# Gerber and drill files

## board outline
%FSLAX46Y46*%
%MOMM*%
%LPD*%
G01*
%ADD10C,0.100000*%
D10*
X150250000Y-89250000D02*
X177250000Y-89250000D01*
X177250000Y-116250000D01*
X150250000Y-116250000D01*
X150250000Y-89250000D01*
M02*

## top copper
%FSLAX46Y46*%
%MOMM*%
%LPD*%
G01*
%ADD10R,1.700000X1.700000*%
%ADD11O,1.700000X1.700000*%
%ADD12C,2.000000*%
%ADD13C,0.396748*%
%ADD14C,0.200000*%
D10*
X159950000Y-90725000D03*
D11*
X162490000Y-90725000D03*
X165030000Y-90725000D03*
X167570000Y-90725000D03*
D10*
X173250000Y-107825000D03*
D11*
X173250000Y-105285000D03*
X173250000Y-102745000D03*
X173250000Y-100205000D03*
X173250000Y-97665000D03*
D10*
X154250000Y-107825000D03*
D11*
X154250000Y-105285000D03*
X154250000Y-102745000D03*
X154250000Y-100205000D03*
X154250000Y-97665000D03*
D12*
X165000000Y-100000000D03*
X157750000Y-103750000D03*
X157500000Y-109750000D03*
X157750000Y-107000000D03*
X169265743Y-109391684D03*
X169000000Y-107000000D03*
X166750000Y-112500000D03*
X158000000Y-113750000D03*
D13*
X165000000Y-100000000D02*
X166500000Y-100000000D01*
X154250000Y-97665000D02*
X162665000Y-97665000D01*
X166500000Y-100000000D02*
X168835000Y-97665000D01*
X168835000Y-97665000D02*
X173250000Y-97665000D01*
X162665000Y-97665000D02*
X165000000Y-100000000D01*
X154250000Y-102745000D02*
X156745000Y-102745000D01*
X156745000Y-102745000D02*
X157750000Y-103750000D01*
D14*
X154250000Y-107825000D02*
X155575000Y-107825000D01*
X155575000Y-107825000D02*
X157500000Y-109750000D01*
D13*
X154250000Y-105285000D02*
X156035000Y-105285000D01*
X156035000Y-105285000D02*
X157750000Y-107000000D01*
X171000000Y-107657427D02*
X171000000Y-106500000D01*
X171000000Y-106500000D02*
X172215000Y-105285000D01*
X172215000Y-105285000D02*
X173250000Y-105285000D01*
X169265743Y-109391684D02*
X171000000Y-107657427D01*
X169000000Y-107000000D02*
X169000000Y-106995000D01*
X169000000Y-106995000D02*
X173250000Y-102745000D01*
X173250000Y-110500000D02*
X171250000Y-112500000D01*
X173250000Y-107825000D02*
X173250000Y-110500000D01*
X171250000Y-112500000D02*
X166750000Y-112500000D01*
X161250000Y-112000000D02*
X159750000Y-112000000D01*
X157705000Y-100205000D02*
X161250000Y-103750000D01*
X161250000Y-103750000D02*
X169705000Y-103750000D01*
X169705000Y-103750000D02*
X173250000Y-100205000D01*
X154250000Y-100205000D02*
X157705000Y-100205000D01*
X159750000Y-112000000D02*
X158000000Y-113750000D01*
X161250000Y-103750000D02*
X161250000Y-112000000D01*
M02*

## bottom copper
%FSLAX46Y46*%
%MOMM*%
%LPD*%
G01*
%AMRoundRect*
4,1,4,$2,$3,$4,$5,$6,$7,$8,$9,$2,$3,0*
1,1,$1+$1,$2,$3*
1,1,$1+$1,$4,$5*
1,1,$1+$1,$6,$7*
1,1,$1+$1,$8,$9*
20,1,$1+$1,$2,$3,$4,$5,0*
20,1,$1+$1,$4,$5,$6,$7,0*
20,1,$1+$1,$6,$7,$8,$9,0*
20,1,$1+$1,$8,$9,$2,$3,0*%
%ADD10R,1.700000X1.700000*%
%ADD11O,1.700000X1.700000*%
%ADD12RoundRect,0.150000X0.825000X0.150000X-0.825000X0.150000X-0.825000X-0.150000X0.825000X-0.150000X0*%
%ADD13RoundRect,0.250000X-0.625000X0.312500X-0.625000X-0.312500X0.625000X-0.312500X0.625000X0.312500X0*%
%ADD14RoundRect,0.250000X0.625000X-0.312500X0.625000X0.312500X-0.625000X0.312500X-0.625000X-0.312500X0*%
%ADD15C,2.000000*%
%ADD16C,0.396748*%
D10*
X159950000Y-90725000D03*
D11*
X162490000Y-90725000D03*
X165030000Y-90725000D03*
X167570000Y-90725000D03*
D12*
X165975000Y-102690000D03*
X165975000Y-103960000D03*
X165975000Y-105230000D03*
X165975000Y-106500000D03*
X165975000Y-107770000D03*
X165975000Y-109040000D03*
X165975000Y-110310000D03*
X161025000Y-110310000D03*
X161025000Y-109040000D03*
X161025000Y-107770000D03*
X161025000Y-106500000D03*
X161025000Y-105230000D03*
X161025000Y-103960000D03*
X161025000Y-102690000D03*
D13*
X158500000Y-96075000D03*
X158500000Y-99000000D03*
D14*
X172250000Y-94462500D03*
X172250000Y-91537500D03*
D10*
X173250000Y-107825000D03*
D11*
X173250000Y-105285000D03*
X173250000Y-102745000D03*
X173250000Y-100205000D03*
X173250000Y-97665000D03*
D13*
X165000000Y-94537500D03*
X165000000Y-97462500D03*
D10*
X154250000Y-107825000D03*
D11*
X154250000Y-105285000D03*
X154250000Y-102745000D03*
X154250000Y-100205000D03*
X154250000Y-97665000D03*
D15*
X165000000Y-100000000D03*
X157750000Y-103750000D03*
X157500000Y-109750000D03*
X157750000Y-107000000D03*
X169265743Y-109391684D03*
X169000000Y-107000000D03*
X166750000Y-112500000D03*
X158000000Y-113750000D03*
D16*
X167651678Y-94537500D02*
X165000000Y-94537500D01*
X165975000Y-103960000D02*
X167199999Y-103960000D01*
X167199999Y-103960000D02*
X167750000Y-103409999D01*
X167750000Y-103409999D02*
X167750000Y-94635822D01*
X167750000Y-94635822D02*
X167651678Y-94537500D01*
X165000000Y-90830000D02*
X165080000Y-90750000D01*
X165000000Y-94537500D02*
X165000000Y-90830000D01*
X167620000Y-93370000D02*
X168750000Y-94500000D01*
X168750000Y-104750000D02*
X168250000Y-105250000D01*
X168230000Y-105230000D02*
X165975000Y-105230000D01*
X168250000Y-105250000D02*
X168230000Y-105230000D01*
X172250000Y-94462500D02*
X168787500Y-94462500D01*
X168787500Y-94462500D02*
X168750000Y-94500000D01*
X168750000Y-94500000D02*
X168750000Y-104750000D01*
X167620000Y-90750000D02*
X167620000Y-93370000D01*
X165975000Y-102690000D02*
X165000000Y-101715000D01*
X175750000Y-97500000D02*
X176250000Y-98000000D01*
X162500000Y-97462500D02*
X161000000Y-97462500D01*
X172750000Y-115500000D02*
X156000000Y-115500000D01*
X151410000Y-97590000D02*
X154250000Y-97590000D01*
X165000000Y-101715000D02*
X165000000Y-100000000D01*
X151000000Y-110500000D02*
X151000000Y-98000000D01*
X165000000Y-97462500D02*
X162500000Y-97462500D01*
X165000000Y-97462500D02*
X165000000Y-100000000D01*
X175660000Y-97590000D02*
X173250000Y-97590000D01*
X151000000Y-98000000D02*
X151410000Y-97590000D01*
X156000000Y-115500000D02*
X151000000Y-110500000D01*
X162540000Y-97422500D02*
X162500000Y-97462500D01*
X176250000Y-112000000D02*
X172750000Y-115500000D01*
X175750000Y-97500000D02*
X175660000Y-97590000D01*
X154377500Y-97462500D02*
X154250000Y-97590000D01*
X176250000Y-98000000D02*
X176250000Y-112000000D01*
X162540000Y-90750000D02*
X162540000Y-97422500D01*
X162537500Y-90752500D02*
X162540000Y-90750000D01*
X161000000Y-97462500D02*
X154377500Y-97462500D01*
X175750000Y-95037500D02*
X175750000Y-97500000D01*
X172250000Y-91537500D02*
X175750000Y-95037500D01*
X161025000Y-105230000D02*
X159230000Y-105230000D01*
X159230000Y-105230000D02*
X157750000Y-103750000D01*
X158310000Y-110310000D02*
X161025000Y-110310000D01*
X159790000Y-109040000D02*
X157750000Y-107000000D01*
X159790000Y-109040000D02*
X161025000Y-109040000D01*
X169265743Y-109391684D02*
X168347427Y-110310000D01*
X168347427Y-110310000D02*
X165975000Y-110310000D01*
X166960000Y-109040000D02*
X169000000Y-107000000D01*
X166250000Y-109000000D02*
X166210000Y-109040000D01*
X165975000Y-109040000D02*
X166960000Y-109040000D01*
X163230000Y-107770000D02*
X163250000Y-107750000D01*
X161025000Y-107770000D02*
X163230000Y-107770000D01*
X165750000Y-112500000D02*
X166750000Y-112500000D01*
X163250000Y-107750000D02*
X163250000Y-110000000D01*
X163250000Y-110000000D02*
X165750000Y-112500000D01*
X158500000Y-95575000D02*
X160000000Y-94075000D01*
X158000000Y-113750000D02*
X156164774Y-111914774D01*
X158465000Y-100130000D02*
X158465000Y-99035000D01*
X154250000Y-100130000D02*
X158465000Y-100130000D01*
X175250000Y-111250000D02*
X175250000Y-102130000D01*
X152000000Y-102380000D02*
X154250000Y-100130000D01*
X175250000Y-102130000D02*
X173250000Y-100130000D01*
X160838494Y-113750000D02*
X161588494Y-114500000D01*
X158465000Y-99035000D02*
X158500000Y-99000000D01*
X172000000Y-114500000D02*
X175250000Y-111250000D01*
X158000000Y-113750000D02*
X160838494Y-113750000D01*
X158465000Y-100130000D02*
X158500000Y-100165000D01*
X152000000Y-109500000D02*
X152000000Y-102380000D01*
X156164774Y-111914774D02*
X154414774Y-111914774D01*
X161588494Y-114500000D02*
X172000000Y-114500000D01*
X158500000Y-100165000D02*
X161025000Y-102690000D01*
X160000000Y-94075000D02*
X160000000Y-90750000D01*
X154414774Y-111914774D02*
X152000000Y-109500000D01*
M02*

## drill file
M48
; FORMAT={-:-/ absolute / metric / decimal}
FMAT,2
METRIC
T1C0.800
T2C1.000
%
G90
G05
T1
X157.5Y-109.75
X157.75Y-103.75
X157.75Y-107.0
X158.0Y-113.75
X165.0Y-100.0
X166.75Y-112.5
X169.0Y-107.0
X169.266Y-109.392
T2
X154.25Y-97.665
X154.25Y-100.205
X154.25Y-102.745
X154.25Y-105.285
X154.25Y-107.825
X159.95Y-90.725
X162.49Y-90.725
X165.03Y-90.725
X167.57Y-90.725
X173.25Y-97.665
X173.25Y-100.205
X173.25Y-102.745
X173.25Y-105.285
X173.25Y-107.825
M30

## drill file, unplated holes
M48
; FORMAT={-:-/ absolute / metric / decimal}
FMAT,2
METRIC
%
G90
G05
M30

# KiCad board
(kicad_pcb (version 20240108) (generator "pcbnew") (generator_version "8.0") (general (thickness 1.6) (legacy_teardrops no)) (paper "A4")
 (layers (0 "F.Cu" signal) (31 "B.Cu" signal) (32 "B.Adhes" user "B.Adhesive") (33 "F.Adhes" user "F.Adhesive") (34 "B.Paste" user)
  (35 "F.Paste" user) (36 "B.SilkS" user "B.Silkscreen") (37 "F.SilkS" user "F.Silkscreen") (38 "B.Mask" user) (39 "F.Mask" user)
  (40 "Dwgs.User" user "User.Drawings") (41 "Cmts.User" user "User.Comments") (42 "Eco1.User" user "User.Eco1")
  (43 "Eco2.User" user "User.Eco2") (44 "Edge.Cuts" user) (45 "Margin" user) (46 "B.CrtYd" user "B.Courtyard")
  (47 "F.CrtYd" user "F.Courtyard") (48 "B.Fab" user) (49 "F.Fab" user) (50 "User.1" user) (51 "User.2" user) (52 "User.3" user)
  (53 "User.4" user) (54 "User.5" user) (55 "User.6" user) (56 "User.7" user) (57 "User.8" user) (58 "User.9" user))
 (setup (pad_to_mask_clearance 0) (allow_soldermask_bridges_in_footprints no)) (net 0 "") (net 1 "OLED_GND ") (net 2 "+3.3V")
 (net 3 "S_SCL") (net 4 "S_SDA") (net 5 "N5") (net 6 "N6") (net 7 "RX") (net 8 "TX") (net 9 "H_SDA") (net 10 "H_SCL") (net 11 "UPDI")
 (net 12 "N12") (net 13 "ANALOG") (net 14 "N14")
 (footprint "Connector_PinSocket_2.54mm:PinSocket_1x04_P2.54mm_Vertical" (layer "F.Cu") (at 159.95 90.725 90)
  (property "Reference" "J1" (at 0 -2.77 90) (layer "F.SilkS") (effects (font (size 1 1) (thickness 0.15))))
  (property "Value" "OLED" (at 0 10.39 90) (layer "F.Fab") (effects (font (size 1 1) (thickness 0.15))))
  (pad "1" thru_hole rect (at 0 0 90) (size 1.7 1.7) (drill 1) (layers "*.Cu" "*.Mask") (remove_unused_layers no) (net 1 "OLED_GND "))
  (pad "2" thru_hole oval (at 0 2.54 90) (size 1.7 1.7) (drill 1) (layers "*.Cu" "*.Mask") (remove_unused_layers no) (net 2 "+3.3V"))
  (pad "3" thru_hole oval (at 0 5.08 90) (size 1.7 1.7) (drill 1) (layers "*.Cu" "*.Mask") (remove_unused_layers no) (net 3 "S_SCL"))
  (pad "4" thru_hole oval (at 0 7.62 90) (size 1.7 1.7) (drill 1) (layers "*.Cu" "*.Mask") (remove_unused_layers no) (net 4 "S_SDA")))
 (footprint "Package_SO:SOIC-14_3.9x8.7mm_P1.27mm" (layer "B.Cu") (at 163.5 106.5 180)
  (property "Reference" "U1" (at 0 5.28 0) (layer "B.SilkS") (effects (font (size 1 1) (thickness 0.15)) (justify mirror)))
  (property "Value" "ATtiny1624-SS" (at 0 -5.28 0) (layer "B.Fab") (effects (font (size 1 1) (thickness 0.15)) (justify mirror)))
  (pad "1" smd roundrect (at -2.475 3.81 180) (size 1.95 0.6) (layers "B.Cu" "B.Paste" "B.Mask") (roundrect_rratio 0.25) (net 2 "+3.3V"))
  (pad "2" smd roundrect (at -2.475 2.54 180) (size 1.95 0.6) (layers "B.Cu" "B.Paste" "B.Mask") (roundrect_rratio 0.25) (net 3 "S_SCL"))
  (pad "3" smd roundrect (at -2.475 1.27 180) (size 1.95 0.6) (layers "B.Cu" "B.Paste" "B.Mask") (roundrect_rratio 0.25) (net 4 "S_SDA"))
  (pad "4" smd roundrect (at -2.475 0 180) (size 1.95 0.6) (layers "B.Cu" "B.Paste" "B.Mask") (roundrect_rratio 0.25) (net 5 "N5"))
  (pad "5" smd roundrect (at -2.475 -1.27 180) (size 1.95 0.6) (layers "B.Cu" "B.Paste" "B.Mask") (roundrect_rratio 0.25) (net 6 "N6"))
  (pad "6" smd roundrect (at -2.475 -2.54 180) (size 1.95 0.6) (layers "B.Cu" "B.Paste" "B.Mask") (roundrect_rratio 0.25) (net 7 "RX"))
  (pad "7" smd roundrect (at -2.475 -3.81 180) (size 1.95 0.6) (layers "B.Cu" "B.Paste" "B.Mask") (roundrect_rratio 0.25) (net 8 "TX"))
  (pad "8" smd roundrect (at 2.475 -3.81 180) (size 1.95 0.6) (layers "B.Cu" "B.Paste" "B.Mask") (roundrect_rratio 0.25) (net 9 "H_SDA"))
  (pad "9" smd roundrect (at 2.475 -2.54 180) (size 1.95 0.6) (layers "B.Cu" "B.Paste" "B.Mask") (roundrect_rratio 0.25) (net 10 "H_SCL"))
  (pad "10" smd roundrect (at 2.475 -1.27 180) (size 1.95 0.6) (layers "B.Cu" "B.Paste" "B.Mask") (roundrect_rratio 0.25) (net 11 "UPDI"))
  (pad "11" smd roundrect (at 2.475 0 180) (size 1.95 0.6) (layers "B.Cu" "B.Paste" "B.Mask") (roundrect_rratio 0.25) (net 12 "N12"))
  (pad "12" smd roundrect (at 2.475 1.27 180) (size 1.95 0.6) (layers "B.Cu" "B.Paste" "B.Mask") (roundrect_rratio 0.25) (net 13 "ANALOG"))
  (pad "13" smd roundrect (at 2.475 2.54 180) (size 1.95 0.6) (layers "B.Cu" "B.Paste" "B.Mask") (roundrect_rratio 0.25) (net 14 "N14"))
  (pad "14" smd roundrect (at 2.475 3.81 180) (size 1.95 0.6) (layers "B.Cu" "B.Paste" "B.Mask") (roundrect_rratio 0.25) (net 1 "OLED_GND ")))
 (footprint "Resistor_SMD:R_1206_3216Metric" (layer "B.Cu") (at 158.5 97.5375 -90)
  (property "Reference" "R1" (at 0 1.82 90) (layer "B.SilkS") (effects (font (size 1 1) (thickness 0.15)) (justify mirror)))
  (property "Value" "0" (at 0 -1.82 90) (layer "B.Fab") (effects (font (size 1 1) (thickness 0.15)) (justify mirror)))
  (pad "1" smd roundrect (at -1.4625 0 270) (size 1.125 1.75) (layers "B.Cu" "B.Paste" "B.Mask") (roundrect_rratio 0.222222)
   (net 1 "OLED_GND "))
  (pad "2" smd roundrect (at 1.4625 0 270) (size 1.125 1.75) (layers "B.Cu" "B.Paste" "B.Mask") (roundrect_rratio 0.222222)
   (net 1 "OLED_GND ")))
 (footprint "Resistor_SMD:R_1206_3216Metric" (layer "B.Cu") (at 172.25 93 90)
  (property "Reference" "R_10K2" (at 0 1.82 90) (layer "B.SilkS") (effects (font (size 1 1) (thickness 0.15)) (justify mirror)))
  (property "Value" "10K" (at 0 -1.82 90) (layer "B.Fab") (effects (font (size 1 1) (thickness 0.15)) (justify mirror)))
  (pad "1" smd roundrect (at -1.4625 0 90) (size 1.125 1.75) (layers "B.Cu" "B.Paste" "B.Mask") (roundrect_rratio 0.222222) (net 4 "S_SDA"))
  (pad "2" smd roundrect (at 1.4625 0 90) (size 1.125 1.75) (layers "B.Cu" "B.Paste" "B.Mask") (roundrect_rratio 0.222222) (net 2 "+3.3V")))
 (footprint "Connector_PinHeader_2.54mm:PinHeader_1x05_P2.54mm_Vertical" (layer "B.Cu") (at 173.25 107.825)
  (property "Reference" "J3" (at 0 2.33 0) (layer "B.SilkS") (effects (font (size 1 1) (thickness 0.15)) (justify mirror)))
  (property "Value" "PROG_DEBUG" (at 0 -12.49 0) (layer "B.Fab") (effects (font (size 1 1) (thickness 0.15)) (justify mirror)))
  (pad "1" thru_hole rect (at 0 0) (size 1.7 1.7) (drill 1) (layers "*.Cu" "*.Mask") (remove_unused_layers no) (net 11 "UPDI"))
  (pad "2" thru_hole oval (at 0 -2.54) (size 1.7 1.7) (drill 1) (layers "*.Cu" "*.Mask") (remove_unused_layers no) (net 8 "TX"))
  (pad "3" thru_hole oval (at 0 -5.08) (size 1.7 1.7) (drill 1) (layers "*.Cu" "*.Mask") (remove_unused_layers no) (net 7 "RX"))
  (pad "4" thru_hole oval (at 0 -7.62) (size 1.7 1.7) (drill 1) (layers "*.Cu" "*.Mask") (remove_unused_layers no) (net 1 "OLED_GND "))
  (pad "5" thru_hole oval (at 0 -10.16) (size 1.7 1.7) (drill 1) (layers "*.Cu" "*.Mask") (remove_unused_layers no) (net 2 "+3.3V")))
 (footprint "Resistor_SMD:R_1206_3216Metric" (layer "B.Cu") (at 165 96 -90)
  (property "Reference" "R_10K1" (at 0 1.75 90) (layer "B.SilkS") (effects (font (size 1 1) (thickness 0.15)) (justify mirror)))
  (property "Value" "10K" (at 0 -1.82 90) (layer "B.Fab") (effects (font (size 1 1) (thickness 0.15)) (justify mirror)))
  (pad "1" smd roundrect (at -1.4625 0 270) (size 1.125 1.75) (layers "B.Cu" "B.Paste" "B.Mask") (roundrect_rratio 0.222222) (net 3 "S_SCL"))
  (pad "2" smd roundrect (at 1.4625 0 270) (size 1.125 1.75) (layers "B.Cu" "B.Paste" "B.Mask") (roundrect_rratio 0.222222) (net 2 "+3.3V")))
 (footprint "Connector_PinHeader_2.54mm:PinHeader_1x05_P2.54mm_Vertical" (layer "B.Cu") (at 154.25 107.825)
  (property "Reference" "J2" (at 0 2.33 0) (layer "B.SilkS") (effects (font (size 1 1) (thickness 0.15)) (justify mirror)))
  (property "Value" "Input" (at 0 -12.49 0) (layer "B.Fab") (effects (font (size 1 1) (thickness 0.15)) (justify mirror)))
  (pad "1" thru_hole rect (at 0 0) (size 1.7 1.7) (drill 1) (layers "*.Cu" "*.Mask") (remove_unused_layers no) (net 9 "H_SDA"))
  (pad "2" thru_hole oval (at 0 -2.54) (size 1.7 1.7) (drill 1) (layers "*.Cu" "*.Mask") (remove_unused_layers no) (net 10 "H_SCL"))
  (pad "3" thru_hole oval (at 0 -5.08) (size 1.7 1.7) (drill 1) (layers "*.Cu" "*.Mask") (remove_unused_layers no) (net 13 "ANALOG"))
  (pad "4" thru_hole oval (at 0 -7.62) (size 1.7 1.7) (drill 1) (layers "*.Cu" "*.Mask") (remove_unused_layers no) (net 1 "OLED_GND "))
  (pad "5" thru_hole oval (at 0 -10.16) (size 1.7 1.7) (drill 1) (layers "*.Cu" "*.Mask") (remove_unused_layers no) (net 2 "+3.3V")))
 (gr_rect (start 150.25 89.25) (end 177.25 116.25) (stroke (width 0.1) (type default)) (fill none) (layer "Edge.Cuts"))
 (segment (start 167.651678 94.5375) (end 165 94.5375) (width 0.396748) (layer "B.Cu") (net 3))
 (segment (start 165.975 103.96) (end 167.199999 103.96) (width 0.396748) (layer "B.Cu") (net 3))
 (segment (start 167.199999 103.96) (end 167.75 103.409999) (width 0.396748) (layer "B.Cu") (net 3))
 (segment (start 167.75 103.409999) (end 167.75 94.635822) (width 0.396748) (layer "B.Cu") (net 3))
 (segment (start 167.75 94.635822) (end 167.651678 94.5375) (width 0.396748) (layer "B.Cu") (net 3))
 (segment (start 165 90.83) (end 165.08 90.75) (width 0.396748) (layer "B.Cu") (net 3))
 (segment (start 165 94.5375) (end 165 90.83) (width 0.396748) (layer "B.Cu") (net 3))
 (segment (start 167.62 93.37) (end 168.75 94.5) (width 0.396748) (layer "B.Cu") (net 4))
 (segment (start 168.75 104.75) (end 168.25 105.25) (width 0.396748) (layer "B.Cu") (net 4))
 (segment (start 168.23 105.23) (end 165.975 105.23) (width 0.396748) (layer "B.Cu") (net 4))
 (segment (start 168.25 105.25) (end 168.23 105.23) (width 0.396748) (layer "B.Cu") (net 4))
 (segment (start 172.25 94.4625) (end 168.7875 94.4625) (width 0.396748) (layer "B.Cu") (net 4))
 (segment (start 168.7875 94.4625) (end 168.75 94.5) (width 0.396748) (layer "B.Cu") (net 4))
 (segment (start 168.75 94.5) (end 168.75 104.75) (width 0.396748) (layer "B.Cu") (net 4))
 (segment (start 167.62 90.75) (end 167.62 93.37) (width 0.396748) (layer "B.Cu") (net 4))
 (segment (start 165 100) (end 166.5 100) (width 0.396748) (layer "F.Cu") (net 2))
 (segment (start 154.25 97.665) (end 162.665 97.665) (width 0.396748) (layer "F.Cu") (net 2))
 (segment (start 166.5 100) (end 168.835 97.665) (width 0.396748) (layer "F.Cu") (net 2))
 (segment (start 168.835 97.665) (end 173.25 97.665) (width 0.396748) (layer "F.Cu") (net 2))
 (segment (start 162.665 97.665) (end 165 100) (width 0.396748) (layer "F.Cu") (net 2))
 (via (at 165 100) (size 2) (drill 0.8) (layers "F.Cu" "B.Cu") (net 2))
 (segment (start 165.975 102.69) (end 165 101.715) (width 0.396748) (layer "B.Cu") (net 2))
 (segment (start 175.75 97.5) (end 176.25 98) (width 0.396748) (layer "B.Cu") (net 2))
 (segment (start 162.5 97.4625) (end 161 97.4625) (width 0.396748) (layer "B.Cu") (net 2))
 (segment (start 172.75 115.5) (end 156 115.5) (width 0.396748) (layer "B.Cu") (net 2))
 (segment (start 151.41 97.59) (end 154.25 97.59) (width 0.396748) (layer "B.Cu") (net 2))
 (segment (start 165 101.715) (end 165 100) (width 0.396748) (layer "B.Cu") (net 2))
 (segment (start 151 110.5) (end 151 98) (width 0.396748) (layer "B.Cu") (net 2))
 (segment (start 165 97.4625) (end 162.5 97.4625) (width 0.396748) (layer "B.Cu") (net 2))
 (segment (start 165 97.4625) (end 165 100) (width 0.396748) (layer "B.Cu") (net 2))
 (segment (start 175.66 97.59) (end 173.25 97.59) (width 0.396748) (layer "B.Cu") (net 2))
 (segment (start 151 98) (end 151.41 97.59) (width 0.396748) (layer "B.Cu") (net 2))
 (segment (start 156 115.5) (end 151 110.5) (width 0.396748) (layer "B.Cu") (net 2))
 (segment (start 162.54 97.4225) (end 162.5 97.4625) (width 0.396748) (layer "B.Cu") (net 2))
 (segment (start 176.25 112) (end 172.75 115.5) (width 0.396748) (layer "B.Cu") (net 2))
 (segment (start 175.75 97.5) (end 175.66 97.59) (width 0.396748) (layer "B.Cu") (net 2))
 (segment (start 154.3775 97.4625) (end 154.25 97.59) (width 0.396748) (layer "B.Cu") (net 2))
 (segment (start 176.25 98) (end 176.25 112) (width 0.396748) (layer "B.Cu") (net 2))
 (segment (start 162.54 90.75) (end 162.54 97.4225) (width 0.396748) (layer "B.Cu") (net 2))
 (segment (start 162.5375 90.7525) (end 162.54 90.75) (width 0.396748) (layer "B.Cu") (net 2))
 (segment (start 161 97.4625) (end 154.3775 97.4625) (width 0.396748) (layer "B.Cu") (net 2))
 (segment (start 175.75 95.0375) (end 175.75 97.5) (width 0.396748) (layer "B.Cu") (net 2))
 (segment (start 172.25 91.5375) (end 175.75 95.0375) (width 0.396748) (layer "B.Cu") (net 2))
 (segment (start 154.25 102.745) (end 156.745 102.745) (width 0.396748) (layer "F.Cu") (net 13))
 (segment (start 156.745 102.745) (end 157.75 103.75) (width 0.396748) (layer "F.Cu") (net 13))
 (via (at 157.75 103.75) (size 2) (drill 0.8) (layers "F.Cu" "B.Cu") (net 13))
 (segment (start 161.025 105.23) (end 159.23 105.23) (width 0.396748) (layer "B.Cu") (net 13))
 (segment (start 159.23 105.23) (end 157.75 103.75) (width 0.396748) (layer "B.Cu") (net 13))
 (segment (start 154.25 107.825) (end 155.575 107.825) (width 0.396748) (layer "F.Cu") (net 9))
 (segment (start 155.575 107.825) (end 157.5 109.75) (width 0.396748) (layer "F.Cu") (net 9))
 (via (at 157.5 109.75) (size 2) (drill 0.8) (layers "F.Cu" "B.Cu") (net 9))
 (segment (start 158.31 110.31) (end 161.025 110.31) (width 0.396748) (layer "B.Cu") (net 9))
 (segment (start 154.25 105.285) (end 156.035 105.285) (width 0.396748) (layer "F.Cu") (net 10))
 (segment (start 156.035 105.285) (end 157.75 107) (width 0.396748) (layer "F.Cu") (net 10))
 (via (at 157.75 107) (size 2) (drill 0.8) (layers "F.Cu" "B.Cu") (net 10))
 (segment (start 159.79 109.04) (end 157.75 107) (width 0.396748) (layer "B.Cu") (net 10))
 (segment (start 159.79 109.04) (end 161.025 109.04) (width 0.396748) (layer "B.Cu") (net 10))
 (segment (start 171 107.657427) (end 171 106.5) (width 0.396748) (layer "F.Cu") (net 8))
 (segment (start 171 106.5) (end 172.215 105.285) (width 0.396748) (layer "F.Cu") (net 8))
 (segment (start 172.215 105.285) (end 173.25 105.285) (width 0.396748) (layer "F.Cu") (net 8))
 (segment (start 169.265743 109.391684) (end 171 107.657427) (width 0.396748) (layer "F.Cu") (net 8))
 (via (at 169.265743 109.391684) (size 2) (drill 0.8) (layers "F.Cu" "B.Cu") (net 8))
 (segment (start 169.265743 109.391684) (end 168.347427 110.31) (width 0.396748) (layer "B.Cu") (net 8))
 (segment (start 168.347427 110.31) (end 165.975 110.31) (width 0.396748) (layer "B.Cu") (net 8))
 (segment (start 169 107) (end 169 106.995) (width 0.396748) (layer "F.Cu") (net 7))
 (segment (start 169 106.995) (end 173.25 102.745) (width 0.396748) (layer "F.Cu") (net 7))
 (via (at 169 107) (size 2) (drill 0.8) (layers "F.Cu" "B.Cu") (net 7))
 (segment (start 166.96 109.04) (end 169 107) (width 0.396748) (layer "B.Cu") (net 7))
 (segment (start 166.25 109) (end 166.21 109.04) (width 0.396748) (layer "B.Cu") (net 7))
 (segment (start 165.975 109.04) (end 166.96 109.04) (width 0.396748) (layer "B.Cu") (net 7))
 (segment (start 173.25 110.5) (end 171.25 112.5) (width 0.396748) (layer "F.Cu") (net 11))
 (segment (start 173.25 107.825) (end 173.25 110.5) (width 0.396748) (layer "F.Cu") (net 11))
 (segment (start 171.25 112.5) (end 166.75 112.5) (width 0.396748) (layer "F.Cu") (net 11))
 (via (at 166.75 112.5) (size 2) (drill 0.8) (layers "F.Cu" "B.Cu") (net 11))
 (segment (start 163.23 107.77) (end 163.25 107.75) (width 0.396748) (layer "B.Cu") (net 11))
 (segment (start 161.025 107.77) (end 163.23 107.77) (width 0.396748) (layer "B.Cu") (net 11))
 (segment (start 165.75 112.5) (end 166.75 112.5) (width 0.396748) (layer "B.Cu") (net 11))
 (segment (start 163.25 107.75) (end 163.25 110) (width 0.396748) (layer "B.Cu") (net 11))
 (segment (start 163.25 110) (end 165.75 112.5) (width 0.396748) (layer "B.Cu") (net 11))
 (segment (start 161.25 112) (end 159.75 112) (width 0.396748) (layer "F.Cu") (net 1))
 (segment (start 157.705 100.205) (end 161.25 103.75) (width 0.396748) (layer "F.Cu") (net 1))
 (segment (start 161.25 103.75) (end 169.705 103.75) (width 0.396748) (layer "F.Cu") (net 1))
 (segment (start 169.705 103.75) (end 173.25 100.205) (width 0.396748) (layer "F.Cu") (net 1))
 (segment (start 154.25 100.205) (end 157.705 100.205) (width 0.396748) (layer "F.Cu") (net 1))
 (segment (start 159.75 112) (end 158 113.75) (width 0.396748) (layer "F.Cu") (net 1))
 (segment (start 161.25 103.75) (end 161.25 112) (width 0.396748) (layer "F.Cu") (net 1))
 (via (at 158 113.75) (size 2) (drill 0.8) (layers "F.Cu" "B.Cu") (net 1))
 (segment (start 158.5 95.575) (end 160 94.075) (width 0.396748) (layer "B.Cu") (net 1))
 (segment (start 158 113.75) (end 156.164774 111.914774) (width 0.396748) (layer "B.Cu") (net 1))
 (segment (start 158.465 100.13) (end 158.465 99.035) (width 0.396748) (layer "B.Cu") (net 1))
 (segment (start 154.25 100.13) (end 158.465 100.13) (width 0.396748) (layer "B.Cu") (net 1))
 (segment (start 175.25 111.25) (end 175.25 102.13) (width 0.396748) (layer "B.Cu") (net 1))
 (segment (start 152 102.38) (end 154.25 100.13) (width 0.396748) (layer "B.Cu") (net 1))
 (segment (start 175.25 102.13) (end 173.25 100.13) (width 0.396748) (layer "B.Cu") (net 1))
 (segment (start 160.838494 113.75) (end 161.588494 114.5) (width 0.396748) (layer "B.Cu") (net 1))
 (segment (start 158.465 99.035) (end 158.5 99) (width 0.396748) (layer "B.Cu") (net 1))
 (segment (start 172 114.5) (end 175.25 111.25) (width 0.396748) (layer "B.Cu") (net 1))
 (segment (start 158 113.75) (end 160.838494 113.75) (width 0.396748) (layer "B.Cu") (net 1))
 (segment (start 158.465 100.13) (end 158.5 100.165) (width 0.396748) (layer "B.Cu") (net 1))
 (segment (start 152 109.5) (end 152 102.38) (width 0.396748) (layer "B.Cu") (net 1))
 (segment (start 156.164774 111.914774) (end 154.414774 111.914774) (width 0.396748) (layer "B.Cu") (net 1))
 (segment (start 161.588494 114.5) (end 172 114.5) (width 0.396748) (layer "B.Cu") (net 1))
 (segment (start 158.5 100.165) (end 161.025 102.69) (width 0.396748) (layer "B.Cu") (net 1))
 (segment (start 160 94.075) (end 160 90.75) (width 0.396748) (layer "B.Cu") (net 1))
 (segment (start 154.414774 111.914774) (end 152 109.5) (width 0.396748) (layer "B.Cu") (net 1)))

